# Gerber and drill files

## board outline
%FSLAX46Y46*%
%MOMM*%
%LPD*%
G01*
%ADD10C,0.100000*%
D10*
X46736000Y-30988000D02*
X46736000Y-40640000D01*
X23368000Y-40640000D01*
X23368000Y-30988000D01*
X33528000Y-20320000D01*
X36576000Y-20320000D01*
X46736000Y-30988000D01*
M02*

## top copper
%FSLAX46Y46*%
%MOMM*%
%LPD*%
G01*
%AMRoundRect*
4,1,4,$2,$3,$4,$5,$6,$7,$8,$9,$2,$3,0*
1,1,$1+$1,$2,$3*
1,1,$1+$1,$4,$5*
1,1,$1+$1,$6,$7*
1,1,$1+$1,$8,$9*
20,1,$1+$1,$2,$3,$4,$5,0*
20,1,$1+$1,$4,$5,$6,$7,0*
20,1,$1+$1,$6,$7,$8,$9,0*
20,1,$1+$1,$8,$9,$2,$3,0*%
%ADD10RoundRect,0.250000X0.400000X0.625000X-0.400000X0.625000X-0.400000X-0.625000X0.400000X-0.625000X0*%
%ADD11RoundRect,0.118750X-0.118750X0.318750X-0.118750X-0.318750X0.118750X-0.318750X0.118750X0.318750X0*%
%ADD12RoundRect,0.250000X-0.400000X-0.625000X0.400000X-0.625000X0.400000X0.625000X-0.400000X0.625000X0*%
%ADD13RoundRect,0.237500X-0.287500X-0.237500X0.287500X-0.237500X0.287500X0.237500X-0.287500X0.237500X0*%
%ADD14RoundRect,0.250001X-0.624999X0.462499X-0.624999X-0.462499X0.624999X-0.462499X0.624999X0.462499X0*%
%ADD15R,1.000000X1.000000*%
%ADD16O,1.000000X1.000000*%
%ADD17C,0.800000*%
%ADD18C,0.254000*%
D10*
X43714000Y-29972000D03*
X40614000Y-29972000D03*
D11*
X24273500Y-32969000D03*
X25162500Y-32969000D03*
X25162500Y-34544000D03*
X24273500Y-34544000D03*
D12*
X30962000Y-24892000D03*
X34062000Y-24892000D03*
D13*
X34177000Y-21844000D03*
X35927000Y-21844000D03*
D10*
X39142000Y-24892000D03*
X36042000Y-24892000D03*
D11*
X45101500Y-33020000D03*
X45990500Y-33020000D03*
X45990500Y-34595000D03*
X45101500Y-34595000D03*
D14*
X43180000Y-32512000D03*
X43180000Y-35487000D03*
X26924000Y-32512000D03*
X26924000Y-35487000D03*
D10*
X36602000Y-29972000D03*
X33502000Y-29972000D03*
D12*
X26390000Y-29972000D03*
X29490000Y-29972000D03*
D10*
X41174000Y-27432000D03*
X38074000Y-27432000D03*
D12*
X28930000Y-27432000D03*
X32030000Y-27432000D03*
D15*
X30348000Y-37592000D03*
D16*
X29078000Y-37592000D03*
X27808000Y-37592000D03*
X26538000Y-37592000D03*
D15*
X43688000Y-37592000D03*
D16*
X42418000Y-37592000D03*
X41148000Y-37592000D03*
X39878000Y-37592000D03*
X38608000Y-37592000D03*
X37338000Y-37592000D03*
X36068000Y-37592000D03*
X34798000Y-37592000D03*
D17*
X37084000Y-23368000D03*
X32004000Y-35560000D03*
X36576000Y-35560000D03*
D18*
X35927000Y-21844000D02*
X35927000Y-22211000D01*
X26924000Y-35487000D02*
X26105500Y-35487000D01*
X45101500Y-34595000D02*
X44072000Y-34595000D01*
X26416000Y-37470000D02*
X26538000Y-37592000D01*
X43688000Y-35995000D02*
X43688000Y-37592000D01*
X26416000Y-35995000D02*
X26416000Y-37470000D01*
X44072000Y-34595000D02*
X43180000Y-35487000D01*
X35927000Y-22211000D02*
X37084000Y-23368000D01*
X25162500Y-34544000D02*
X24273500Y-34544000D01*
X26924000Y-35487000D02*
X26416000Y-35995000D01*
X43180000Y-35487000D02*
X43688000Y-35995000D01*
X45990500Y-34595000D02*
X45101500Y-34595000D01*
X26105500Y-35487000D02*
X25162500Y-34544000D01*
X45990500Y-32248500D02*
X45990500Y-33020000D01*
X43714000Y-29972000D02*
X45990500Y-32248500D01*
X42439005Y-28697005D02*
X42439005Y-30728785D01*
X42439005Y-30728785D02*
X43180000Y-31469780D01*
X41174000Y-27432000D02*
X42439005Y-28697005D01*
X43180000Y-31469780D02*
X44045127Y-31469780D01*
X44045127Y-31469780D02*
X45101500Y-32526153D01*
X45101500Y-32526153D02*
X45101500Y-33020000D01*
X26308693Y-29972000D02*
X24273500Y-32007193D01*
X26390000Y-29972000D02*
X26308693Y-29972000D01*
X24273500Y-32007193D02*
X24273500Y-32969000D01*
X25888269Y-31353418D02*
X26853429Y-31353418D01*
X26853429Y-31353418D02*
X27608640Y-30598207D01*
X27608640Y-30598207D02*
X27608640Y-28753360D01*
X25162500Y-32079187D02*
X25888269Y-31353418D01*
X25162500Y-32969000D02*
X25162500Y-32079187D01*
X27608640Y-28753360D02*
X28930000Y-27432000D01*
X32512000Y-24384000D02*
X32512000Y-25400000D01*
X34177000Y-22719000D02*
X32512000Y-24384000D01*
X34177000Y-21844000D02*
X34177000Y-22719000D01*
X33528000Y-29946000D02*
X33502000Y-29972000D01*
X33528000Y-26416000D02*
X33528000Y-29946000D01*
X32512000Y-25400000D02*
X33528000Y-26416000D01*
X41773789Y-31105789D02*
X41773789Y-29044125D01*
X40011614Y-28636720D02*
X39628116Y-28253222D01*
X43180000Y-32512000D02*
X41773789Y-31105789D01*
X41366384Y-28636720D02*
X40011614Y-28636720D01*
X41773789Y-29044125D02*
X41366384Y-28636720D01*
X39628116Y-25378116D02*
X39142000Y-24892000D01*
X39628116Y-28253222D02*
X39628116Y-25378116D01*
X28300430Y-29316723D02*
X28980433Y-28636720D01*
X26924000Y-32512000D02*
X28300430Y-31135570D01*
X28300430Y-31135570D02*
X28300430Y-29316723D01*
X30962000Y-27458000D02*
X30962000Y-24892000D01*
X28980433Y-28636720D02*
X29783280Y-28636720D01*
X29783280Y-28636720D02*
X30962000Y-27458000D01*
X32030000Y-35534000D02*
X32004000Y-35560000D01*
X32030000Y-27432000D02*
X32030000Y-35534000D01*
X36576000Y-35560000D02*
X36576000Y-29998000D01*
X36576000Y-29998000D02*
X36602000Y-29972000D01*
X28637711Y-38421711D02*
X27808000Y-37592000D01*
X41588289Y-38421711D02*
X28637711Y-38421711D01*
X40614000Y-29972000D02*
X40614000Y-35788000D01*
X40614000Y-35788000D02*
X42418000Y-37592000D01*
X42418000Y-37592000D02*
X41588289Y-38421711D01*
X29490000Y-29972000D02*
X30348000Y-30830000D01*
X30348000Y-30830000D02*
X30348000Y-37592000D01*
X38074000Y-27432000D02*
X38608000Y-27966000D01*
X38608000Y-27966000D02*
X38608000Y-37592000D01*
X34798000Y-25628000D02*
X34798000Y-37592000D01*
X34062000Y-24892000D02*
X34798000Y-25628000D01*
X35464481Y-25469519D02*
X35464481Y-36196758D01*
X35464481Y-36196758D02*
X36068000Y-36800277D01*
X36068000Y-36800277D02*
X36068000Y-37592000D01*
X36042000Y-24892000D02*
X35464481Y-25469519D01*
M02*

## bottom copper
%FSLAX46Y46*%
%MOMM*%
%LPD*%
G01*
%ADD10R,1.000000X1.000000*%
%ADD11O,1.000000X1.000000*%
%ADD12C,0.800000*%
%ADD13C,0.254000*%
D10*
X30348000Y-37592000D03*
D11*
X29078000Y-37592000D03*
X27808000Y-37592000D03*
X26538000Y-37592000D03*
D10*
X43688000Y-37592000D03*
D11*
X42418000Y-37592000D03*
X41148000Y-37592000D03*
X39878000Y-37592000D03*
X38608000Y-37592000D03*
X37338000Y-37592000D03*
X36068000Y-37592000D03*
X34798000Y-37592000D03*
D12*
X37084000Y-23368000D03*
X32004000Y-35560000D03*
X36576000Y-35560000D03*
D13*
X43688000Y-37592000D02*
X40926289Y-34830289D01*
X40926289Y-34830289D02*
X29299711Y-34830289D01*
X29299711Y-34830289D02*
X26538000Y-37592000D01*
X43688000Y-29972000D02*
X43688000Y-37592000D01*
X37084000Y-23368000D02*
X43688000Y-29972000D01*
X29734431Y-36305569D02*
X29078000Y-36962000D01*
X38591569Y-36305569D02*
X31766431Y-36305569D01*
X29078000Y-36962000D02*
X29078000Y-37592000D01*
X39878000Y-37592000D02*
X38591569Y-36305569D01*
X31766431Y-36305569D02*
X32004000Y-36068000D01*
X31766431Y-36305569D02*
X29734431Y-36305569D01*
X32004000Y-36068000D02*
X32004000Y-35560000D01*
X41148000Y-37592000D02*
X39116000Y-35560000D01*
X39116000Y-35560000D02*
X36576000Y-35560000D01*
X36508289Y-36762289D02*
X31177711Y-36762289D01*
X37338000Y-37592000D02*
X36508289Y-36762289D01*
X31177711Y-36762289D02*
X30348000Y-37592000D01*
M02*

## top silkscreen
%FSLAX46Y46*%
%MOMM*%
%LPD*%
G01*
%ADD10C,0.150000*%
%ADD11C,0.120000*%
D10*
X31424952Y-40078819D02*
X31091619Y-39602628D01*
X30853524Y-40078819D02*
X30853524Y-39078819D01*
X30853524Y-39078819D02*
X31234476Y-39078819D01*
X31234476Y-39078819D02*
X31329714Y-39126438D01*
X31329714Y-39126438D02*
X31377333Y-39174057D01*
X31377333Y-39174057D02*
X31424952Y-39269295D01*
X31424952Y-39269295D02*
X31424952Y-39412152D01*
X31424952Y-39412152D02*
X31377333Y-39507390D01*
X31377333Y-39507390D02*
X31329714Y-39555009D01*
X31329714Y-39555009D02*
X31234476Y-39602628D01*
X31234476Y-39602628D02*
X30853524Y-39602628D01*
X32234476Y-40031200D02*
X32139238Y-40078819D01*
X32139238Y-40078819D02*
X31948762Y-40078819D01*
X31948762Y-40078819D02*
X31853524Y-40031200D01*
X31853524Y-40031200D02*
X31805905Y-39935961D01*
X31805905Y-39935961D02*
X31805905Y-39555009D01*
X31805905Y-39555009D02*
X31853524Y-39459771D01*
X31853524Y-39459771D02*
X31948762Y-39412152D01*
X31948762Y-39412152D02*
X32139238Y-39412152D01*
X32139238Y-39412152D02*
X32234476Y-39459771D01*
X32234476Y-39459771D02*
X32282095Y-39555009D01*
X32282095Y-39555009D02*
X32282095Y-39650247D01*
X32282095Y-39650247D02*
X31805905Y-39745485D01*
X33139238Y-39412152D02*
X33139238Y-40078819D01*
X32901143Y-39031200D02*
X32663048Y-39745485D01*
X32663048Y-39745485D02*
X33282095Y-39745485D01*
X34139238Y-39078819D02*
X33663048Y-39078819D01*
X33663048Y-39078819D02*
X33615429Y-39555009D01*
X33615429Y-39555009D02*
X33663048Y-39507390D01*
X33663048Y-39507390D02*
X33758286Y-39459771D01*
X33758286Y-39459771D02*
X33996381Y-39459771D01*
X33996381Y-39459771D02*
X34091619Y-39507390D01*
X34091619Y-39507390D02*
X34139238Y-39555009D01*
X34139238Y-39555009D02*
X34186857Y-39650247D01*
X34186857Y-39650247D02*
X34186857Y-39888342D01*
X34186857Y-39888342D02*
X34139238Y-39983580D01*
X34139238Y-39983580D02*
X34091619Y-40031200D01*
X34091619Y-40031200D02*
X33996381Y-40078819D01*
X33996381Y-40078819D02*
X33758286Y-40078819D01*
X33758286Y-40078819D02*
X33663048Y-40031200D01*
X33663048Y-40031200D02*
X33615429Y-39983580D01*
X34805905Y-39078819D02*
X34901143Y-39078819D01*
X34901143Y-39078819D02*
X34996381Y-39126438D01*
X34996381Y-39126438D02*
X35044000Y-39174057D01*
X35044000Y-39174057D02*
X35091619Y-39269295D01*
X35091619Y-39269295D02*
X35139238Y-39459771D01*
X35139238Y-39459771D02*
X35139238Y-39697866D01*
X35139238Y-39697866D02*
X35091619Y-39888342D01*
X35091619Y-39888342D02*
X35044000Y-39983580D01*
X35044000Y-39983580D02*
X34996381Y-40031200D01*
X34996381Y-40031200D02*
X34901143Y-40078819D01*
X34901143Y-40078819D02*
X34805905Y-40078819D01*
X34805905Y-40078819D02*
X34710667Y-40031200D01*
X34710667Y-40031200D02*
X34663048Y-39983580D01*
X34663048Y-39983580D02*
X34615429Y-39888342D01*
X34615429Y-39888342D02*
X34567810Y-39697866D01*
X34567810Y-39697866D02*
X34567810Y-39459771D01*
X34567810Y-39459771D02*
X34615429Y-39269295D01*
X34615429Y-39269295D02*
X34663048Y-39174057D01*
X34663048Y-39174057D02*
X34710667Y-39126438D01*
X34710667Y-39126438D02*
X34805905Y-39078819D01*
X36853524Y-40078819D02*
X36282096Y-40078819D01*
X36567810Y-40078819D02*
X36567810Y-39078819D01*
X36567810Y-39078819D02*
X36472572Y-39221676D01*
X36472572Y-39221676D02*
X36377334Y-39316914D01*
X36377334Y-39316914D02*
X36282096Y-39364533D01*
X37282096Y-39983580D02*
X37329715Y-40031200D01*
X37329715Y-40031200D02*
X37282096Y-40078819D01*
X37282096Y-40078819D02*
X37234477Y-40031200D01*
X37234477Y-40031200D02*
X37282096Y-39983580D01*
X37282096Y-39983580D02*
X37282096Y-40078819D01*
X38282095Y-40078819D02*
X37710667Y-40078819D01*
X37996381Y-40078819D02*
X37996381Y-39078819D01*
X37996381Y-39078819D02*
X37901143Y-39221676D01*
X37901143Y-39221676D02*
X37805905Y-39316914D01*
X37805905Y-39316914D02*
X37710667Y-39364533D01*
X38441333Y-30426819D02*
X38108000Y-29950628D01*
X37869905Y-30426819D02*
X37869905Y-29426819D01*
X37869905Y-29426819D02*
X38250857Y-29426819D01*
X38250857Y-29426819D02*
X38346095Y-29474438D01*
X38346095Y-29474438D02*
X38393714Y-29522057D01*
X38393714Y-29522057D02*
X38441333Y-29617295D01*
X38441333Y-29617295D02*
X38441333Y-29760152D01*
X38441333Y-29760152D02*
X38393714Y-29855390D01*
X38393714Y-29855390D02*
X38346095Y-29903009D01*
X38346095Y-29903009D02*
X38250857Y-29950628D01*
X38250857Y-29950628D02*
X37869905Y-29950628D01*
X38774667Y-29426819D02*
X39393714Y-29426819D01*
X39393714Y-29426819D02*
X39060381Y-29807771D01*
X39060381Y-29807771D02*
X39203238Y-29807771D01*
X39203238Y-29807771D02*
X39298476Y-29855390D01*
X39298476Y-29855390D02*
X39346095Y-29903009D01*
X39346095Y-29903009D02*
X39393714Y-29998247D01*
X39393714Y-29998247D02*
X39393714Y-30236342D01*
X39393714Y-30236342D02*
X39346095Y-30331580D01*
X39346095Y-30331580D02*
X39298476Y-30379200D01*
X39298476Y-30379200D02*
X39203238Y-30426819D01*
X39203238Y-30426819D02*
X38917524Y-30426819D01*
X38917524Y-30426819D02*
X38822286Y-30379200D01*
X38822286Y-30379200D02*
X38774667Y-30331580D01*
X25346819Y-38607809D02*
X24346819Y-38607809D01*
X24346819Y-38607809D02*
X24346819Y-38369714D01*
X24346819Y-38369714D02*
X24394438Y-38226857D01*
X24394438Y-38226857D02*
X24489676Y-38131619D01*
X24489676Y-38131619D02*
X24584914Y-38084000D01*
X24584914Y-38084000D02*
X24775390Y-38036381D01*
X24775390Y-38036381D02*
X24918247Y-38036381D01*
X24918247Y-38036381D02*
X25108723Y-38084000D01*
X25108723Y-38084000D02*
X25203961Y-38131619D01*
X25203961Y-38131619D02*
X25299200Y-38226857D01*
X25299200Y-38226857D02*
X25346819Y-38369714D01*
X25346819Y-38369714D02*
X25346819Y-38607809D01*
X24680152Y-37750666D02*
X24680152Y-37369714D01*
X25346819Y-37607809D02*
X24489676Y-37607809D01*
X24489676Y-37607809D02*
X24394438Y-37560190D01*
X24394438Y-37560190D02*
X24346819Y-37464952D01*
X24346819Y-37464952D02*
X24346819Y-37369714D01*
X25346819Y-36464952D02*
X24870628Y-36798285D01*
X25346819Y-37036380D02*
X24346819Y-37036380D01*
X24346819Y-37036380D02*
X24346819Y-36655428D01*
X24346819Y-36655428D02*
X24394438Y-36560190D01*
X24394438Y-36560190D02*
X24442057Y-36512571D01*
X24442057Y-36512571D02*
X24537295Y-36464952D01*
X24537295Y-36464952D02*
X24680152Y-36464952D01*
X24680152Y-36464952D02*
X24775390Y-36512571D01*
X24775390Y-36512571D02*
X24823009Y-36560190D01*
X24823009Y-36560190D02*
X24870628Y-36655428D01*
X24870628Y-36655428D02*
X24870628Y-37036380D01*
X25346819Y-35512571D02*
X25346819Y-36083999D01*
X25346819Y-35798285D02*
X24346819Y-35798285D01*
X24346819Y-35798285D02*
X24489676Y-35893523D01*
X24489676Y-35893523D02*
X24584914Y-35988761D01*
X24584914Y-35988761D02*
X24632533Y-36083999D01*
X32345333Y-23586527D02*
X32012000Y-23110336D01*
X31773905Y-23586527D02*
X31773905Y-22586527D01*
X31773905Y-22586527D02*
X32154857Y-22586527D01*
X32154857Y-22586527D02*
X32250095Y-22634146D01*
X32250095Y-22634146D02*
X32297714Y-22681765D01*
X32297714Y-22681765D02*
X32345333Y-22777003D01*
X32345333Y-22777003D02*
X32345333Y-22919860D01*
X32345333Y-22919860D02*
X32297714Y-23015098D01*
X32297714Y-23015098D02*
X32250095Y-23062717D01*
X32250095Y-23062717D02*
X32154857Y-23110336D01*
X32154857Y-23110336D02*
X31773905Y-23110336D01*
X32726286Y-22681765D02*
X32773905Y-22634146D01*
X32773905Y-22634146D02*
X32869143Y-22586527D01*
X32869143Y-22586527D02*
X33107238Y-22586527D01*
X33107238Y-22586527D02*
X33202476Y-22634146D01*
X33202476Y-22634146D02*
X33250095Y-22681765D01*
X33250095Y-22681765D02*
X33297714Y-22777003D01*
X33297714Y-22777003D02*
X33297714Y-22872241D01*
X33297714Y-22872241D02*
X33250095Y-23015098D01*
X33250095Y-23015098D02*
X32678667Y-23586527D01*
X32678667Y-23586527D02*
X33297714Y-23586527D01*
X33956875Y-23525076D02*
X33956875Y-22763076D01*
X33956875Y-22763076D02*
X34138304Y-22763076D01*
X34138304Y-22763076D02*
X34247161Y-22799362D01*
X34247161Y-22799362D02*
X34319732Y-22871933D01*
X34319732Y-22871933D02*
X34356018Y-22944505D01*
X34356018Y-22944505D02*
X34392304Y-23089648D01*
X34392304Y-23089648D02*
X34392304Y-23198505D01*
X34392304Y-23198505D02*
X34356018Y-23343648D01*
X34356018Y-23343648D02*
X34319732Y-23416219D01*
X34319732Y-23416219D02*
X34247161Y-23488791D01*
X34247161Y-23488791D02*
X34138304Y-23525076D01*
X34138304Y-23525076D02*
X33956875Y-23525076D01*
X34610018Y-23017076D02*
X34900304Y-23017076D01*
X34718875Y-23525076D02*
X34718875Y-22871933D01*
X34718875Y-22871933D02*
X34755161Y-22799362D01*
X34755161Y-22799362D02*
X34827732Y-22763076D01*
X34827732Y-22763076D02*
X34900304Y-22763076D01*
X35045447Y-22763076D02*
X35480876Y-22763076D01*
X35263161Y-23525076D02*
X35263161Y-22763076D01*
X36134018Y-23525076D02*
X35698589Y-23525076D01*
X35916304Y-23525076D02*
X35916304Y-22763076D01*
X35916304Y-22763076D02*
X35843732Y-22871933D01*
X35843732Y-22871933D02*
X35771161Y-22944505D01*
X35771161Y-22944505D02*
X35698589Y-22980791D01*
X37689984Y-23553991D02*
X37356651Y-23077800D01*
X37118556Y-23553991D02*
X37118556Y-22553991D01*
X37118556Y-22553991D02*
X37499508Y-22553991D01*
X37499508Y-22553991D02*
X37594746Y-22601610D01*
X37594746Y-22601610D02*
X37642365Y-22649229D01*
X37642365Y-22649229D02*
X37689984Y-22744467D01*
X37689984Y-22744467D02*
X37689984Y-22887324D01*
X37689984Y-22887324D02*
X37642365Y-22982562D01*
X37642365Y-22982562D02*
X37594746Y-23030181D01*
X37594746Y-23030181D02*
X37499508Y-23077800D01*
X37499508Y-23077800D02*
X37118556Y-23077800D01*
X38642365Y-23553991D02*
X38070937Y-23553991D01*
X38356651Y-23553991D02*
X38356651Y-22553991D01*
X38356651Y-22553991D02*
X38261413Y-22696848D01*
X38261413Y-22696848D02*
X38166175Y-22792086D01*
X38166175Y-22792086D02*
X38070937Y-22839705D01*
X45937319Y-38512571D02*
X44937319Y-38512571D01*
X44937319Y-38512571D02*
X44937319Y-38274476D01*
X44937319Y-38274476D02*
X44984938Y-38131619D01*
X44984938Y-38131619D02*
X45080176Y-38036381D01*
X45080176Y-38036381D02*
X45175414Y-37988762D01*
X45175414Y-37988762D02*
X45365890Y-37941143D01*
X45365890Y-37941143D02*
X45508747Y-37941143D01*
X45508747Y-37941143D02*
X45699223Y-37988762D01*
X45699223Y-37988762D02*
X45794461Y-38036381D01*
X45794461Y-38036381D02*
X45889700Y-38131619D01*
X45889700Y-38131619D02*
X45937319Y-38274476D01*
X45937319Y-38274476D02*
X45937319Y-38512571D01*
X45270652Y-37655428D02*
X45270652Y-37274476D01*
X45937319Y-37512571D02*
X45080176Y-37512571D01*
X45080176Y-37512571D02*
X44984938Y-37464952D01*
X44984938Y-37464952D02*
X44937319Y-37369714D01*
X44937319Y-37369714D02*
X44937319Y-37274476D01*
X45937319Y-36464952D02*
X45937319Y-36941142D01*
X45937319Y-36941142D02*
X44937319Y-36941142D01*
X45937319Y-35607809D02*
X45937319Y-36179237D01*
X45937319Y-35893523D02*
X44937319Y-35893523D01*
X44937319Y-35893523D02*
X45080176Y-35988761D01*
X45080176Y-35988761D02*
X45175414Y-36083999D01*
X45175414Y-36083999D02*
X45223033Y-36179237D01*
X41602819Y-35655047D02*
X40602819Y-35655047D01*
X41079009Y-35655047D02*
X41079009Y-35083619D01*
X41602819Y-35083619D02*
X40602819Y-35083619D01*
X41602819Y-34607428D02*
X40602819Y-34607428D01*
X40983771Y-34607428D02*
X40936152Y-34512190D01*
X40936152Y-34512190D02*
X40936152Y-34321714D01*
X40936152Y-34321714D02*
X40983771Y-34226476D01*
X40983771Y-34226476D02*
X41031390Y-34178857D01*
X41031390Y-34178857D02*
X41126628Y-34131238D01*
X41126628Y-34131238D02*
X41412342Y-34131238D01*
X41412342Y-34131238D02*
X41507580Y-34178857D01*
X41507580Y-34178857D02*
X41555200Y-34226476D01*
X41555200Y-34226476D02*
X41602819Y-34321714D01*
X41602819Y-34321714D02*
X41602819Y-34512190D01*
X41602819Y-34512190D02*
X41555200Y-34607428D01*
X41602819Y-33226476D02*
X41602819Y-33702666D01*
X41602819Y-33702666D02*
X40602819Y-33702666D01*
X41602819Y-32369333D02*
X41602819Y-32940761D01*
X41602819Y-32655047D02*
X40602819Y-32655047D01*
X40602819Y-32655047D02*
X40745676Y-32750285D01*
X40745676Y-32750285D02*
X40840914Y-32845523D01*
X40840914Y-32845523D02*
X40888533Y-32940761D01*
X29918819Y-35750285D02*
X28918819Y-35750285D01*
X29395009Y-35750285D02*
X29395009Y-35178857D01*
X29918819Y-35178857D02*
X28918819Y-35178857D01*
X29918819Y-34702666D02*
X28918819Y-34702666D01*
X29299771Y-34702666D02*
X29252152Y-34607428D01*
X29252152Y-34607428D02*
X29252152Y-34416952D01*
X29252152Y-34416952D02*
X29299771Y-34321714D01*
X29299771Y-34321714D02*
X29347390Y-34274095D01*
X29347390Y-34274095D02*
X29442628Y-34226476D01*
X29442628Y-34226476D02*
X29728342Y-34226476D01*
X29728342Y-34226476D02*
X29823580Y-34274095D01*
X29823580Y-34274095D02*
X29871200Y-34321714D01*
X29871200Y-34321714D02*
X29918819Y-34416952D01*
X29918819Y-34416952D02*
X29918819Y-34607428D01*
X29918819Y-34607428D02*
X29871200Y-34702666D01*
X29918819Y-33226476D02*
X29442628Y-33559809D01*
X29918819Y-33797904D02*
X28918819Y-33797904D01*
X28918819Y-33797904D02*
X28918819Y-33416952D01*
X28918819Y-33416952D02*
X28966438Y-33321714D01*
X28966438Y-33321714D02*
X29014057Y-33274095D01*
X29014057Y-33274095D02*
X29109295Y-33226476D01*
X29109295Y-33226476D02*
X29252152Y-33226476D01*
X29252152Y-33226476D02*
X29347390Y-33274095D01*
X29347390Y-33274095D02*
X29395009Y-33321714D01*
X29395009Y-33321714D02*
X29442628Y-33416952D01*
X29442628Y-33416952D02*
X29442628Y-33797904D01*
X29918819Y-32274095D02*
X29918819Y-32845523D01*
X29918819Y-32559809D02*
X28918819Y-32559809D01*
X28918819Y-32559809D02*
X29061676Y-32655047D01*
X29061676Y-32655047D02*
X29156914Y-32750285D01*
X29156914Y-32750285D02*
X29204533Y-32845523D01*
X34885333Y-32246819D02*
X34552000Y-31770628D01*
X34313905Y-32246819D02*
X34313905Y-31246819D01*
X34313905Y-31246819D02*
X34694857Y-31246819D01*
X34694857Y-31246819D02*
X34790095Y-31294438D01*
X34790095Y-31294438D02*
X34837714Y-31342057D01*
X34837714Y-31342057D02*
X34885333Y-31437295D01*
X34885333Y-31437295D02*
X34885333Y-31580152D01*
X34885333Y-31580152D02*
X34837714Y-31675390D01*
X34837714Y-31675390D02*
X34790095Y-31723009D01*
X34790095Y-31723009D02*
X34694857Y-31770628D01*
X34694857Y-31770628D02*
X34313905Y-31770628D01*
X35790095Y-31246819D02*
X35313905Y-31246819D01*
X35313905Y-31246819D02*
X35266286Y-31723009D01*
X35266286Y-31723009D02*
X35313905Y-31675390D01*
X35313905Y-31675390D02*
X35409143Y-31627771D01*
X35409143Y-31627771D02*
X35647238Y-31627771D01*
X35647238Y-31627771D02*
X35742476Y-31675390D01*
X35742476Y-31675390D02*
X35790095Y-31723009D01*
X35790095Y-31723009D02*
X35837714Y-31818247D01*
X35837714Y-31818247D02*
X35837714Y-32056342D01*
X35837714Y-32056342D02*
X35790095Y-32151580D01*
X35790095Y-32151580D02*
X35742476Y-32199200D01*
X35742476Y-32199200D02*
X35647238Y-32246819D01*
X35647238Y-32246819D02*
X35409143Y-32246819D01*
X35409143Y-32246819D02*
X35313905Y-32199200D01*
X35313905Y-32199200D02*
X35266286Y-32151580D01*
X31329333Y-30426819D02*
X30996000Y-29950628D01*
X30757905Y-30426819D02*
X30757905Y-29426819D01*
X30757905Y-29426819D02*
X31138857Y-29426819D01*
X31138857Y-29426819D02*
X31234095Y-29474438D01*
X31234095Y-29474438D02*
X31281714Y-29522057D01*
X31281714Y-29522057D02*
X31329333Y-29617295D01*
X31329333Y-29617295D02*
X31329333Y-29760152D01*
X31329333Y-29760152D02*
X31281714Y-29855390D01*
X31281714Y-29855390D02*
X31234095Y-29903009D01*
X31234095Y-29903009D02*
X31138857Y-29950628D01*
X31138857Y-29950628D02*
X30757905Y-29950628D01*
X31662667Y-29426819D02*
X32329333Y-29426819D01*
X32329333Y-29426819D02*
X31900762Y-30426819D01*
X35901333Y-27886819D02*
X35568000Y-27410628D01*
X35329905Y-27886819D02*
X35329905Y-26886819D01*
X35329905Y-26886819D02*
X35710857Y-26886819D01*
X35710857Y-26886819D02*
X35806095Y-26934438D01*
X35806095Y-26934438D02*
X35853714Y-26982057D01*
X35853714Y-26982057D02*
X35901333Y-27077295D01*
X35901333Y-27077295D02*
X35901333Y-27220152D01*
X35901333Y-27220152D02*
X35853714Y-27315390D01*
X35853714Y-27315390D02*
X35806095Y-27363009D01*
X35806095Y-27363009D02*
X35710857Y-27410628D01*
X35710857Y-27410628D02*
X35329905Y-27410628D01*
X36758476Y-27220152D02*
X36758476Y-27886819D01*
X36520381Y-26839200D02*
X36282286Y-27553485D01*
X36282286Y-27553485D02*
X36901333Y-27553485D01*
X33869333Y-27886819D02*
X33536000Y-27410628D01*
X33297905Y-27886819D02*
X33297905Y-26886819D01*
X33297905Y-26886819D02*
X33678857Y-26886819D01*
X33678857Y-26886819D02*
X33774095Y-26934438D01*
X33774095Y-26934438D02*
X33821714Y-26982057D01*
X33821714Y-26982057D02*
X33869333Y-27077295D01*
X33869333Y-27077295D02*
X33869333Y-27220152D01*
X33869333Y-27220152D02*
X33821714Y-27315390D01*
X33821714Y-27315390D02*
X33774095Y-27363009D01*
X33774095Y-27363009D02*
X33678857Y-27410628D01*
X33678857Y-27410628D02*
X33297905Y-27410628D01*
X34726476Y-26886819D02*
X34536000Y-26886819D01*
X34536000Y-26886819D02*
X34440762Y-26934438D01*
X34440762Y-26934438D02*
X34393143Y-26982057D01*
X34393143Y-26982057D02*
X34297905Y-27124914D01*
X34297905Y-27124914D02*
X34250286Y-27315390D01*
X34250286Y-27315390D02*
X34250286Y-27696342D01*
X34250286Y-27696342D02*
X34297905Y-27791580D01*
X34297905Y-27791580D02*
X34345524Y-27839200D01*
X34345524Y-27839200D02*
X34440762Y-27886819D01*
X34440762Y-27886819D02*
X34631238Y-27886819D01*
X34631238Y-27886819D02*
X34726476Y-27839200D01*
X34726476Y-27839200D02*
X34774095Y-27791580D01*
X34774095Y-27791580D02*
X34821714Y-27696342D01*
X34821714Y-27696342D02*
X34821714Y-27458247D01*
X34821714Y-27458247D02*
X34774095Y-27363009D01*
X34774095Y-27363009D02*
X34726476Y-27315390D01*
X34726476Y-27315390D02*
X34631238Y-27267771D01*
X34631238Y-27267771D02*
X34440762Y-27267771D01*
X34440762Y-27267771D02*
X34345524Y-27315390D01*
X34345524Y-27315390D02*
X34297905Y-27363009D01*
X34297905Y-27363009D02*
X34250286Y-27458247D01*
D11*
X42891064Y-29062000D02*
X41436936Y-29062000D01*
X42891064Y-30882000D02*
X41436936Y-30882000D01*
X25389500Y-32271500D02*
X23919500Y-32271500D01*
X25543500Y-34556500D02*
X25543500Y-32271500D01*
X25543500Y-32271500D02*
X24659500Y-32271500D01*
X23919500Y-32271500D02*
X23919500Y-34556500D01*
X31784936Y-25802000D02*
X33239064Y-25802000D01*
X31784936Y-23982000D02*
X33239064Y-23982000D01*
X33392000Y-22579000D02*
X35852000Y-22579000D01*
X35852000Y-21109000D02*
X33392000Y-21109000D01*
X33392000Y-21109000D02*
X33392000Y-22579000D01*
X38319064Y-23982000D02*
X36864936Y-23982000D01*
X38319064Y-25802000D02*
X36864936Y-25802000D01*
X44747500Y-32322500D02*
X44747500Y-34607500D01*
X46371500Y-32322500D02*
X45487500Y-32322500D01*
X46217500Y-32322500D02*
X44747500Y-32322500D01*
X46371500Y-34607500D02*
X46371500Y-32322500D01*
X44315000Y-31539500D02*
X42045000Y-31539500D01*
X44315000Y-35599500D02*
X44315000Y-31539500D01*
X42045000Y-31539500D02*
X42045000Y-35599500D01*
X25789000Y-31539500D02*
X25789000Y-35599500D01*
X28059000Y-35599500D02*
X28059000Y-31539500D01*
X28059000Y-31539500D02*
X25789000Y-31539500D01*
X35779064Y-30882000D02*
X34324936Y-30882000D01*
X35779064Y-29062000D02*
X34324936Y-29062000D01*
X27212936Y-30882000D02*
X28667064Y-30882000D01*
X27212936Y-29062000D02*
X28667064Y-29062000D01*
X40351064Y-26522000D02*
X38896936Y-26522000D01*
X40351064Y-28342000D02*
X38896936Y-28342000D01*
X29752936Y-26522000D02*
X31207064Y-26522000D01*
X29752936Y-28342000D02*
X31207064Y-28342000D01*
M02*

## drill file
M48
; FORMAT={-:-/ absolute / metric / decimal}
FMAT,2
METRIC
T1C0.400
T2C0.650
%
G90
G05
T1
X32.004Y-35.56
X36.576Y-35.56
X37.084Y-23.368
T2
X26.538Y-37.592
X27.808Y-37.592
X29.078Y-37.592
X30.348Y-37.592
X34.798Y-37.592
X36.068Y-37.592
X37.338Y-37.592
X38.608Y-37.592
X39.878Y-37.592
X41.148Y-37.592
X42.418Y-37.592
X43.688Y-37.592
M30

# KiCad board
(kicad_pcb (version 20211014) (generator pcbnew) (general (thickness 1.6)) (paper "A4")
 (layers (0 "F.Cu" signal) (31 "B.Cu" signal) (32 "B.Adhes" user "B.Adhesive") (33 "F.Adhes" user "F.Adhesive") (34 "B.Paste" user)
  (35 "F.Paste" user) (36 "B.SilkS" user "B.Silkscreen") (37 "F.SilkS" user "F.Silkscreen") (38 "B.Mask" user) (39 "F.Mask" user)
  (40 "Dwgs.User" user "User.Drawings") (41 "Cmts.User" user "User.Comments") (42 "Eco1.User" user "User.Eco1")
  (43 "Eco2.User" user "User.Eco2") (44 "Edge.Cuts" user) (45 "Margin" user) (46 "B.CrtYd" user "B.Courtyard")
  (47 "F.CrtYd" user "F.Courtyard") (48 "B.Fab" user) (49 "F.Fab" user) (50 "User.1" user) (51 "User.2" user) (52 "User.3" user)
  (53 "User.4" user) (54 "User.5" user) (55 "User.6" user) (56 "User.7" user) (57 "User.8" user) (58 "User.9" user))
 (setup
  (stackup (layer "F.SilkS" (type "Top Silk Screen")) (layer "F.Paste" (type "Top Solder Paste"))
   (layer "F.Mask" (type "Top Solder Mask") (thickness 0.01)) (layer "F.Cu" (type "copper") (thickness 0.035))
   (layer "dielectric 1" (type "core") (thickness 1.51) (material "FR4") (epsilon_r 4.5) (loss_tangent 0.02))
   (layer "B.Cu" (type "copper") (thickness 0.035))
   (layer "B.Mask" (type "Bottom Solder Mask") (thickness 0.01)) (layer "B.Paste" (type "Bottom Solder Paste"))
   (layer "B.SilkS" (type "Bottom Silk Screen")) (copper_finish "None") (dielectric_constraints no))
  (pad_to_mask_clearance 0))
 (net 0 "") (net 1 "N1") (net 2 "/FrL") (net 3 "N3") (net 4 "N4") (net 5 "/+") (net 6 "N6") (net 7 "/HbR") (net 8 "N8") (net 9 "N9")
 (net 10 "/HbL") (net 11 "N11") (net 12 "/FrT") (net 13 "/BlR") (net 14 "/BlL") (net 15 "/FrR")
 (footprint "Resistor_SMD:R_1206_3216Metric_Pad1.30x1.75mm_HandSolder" (layer "F.Cu") (at 42.164 29.972 180)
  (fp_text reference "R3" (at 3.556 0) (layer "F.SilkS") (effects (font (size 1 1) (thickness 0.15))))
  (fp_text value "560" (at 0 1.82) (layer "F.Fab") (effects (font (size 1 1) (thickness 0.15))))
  (fp_line (start -0.727064 0.91) (end 0.727064 0.91) (layer "F.SilkS") (width 0.12))
  (fp_line (start -0.727064 -0.91) (end 0.727064 -0.91) (layer "F.SilkS") (width 0.12))
  (pad "1" smd roundrect (at -1.55 0 180) (size 1.3 1.75) (layers "F.Cu" "F.Paste" "F.Mask") (roundrect_rratio 0.192308) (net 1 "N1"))
  (pad "2" smd roundrect (at 1.55 0 180) (size 1.3 1.75) (layers "F.Cu" "F.Paste" "F.Mask") (roundrect_rratio 0.192308) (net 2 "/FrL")))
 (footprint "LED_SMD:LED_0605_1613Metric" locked (layer "F.Cu") (at 24.6545 33.7565 -90)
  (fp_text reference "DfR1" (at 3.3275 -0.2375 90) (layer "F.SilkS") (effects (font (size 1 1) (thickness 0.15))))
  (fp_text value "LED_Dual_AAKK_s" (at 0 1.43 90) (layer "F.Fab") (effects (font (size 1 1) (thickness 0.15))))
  (fp_line (start -1.485 -0.735) (end -1.485 0.735) (layer "F.SilkS") (width 0.12))
  (fp_line (start 0.8 -0.889) (end -1.485 -0.889) (layer "F.SilkS") (width 0.12))
  (fp_line (start -1.485 -0.889) (end -1.485 -0.005) (layer "F.SilkS") (width 0.12))
  (fp_line (start -1.485 0.735) (end 0.8 0.735) (layer "F.SilkS") (width 0.12))
  (pad "1" smd roundrect locked (at -0.7875 0.381 270) (size 0.875 0.475) (layers "F.Cu" "F.Paste" "F.Mask") (roundrect_rratio 0.25)
   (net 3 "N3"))
  (pad "2" smd roundrect locked (at -0.7875 -0.508 270) (size 0.875 0.475) (layers "F.Cu" "F.Paste" "F.Mask") (roundrect_rratio 0.25)
   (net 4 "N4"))
  (pad "3" smd roundrect locked (at 0.7875 -0.508 270) (size 0.875 0.475) (layers "F.Cu" "F.Paste" "F.Mask") (roundrect_rratio 0.25)
   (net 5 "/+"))
  (pad "4" smd roundrect locked (at 0.7875 0.381 270) (size 0.875 0.475) (layers "F.Cu" "F.Paste" "F.Mask") (roundrect_rratio 0.25)
   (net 5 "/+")))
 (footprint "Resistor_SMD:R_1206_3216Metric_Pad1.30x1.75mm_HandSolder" (layer "F.Cu") (at 32.512 24.892)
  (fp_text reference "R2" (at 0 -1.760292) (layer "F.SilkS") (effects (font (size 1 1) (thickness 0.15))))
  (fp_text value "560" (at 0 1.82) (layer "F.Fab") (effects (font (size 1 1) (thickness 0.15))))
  (fp_line (start -0.727064 0.91) (end 0.727064 0.91) (layer "F.SilkS") (width 0.12))
  (fp_line (start -0.727064 -0.91) (end 0.727064 -0.91) (layer "F.SilkS") (width 0.12))
  (pad "1" smd roundrect (at -1.55 0) (size 1.3 1.75) (layers "F.Cu" "F.Paste" "F.Mask") (roundrect_rratio 0.192308) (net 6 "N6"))
  (pad "2" smd roundrect (at 1.55 0) (size 1.3 1.75) (layers "F.Cu" "F.Paste" "F.Mask") (roundrect_rratio 0.192308) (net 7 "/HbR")))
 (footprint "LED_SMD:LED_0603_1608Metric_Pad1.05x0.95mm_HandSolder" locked (layer "F.Cu") (at 35.052 21.844)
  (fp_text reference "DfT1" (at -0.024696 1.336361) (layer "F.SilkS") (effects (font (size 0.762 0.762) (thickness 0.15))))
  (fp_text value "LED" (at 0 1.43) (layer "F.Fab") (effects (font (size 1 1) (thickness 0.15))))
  (fp_line (start -1.66 0.735) (end 0.8 0.735) (layer "F.SilkS") (width 0.12))
  (fp_line (start 0.8 -0.735) (end -1.66 -0.735) (layer "F.SilkS") (width 0.12))
  (fp_line (start -1.66 -0.735) (end -1.66 0.735) (layer "F.SilkS") (width 0.12))
  (pad "1" smd roundrect locked (at -0.875 0) (size 1.05 0.95) (layers "F.Cu" "F.Paste" "F.Mask") (roundrect_rratio 0.25) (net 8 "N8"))
  (pad "2" smd roundrect locked (at 0.875 0) (size 1.05 0.95) (layers "F.Cu" "F.Paste" "F.Mask") (roundrect_rratio 0.25) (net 5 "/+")))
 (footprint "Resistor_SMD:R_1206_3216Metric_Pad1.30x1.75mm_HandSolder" (layer "F.Cu") (at 37.592 24.892 180)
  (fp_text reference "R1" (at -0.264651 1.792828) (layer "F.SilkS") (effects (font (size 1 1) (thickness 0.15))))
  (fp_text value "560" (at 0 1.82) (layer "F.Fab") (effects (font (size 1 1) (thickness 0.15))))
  (fp_line (start -0.727064 0.91) (end 0.727064 0.91) (layer "F.SilkS") (width 0.12))
  (fp_line (start -0.727064 -0.91) (end 0.727064 -0.91) (layer "F.SilkS") (width 0.12))
  (pad "1" smd roundrect (at -1.55 0 180) (size 1.3 1.75) (layers "F.Cu" "F.Paste" "F.Mask") (roundrect_rratio 0.192308) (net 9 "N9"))
  (pad "2" smd roundrect (at 1.55 0 180) (size 1.3 1.75) (layers "F.Cu" "F.Paste" "F.Mask") (roundrect_rratio 0.192308) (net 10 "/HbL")))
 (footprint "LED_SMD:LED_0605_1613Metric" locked (layer "F.Cu") (at 45.4825 33.8075 -90)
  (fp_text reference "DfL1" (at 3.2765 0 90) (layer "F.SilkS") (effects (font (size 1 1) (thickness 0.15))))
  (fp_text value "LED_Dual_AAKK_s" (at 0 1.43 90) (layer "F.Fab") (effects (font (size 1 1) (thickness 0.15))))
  (fp_line (start -1.485 0.735) (end 0.8 0.735) (layer "F.SilkS") (width 0.12))
  (fp_line (start -1.485 -0.889) (end -1.485 -0.005) (layer "F.SilkS") (width 0.12))
  (fp_line (start -1.485 -0.735) (end -1.485 0.735) (layer "F.SilkS") (width 0.12))
  (fp_line (start 0.8 -0.889) (end -1.485 -0.889) (layer "F.SilkS") (width 0.12))
  (pad "1" smd roundrect locked (at -0.7875 0.381 270) (size 0.875 0.475) (layers "F.Cu" "F.Paste" "F.Mask") (roundrect_rratio 0.25)
   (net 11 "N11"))
  (pad "2" smd roundrect locked (at -0.7875 -0.508 270) (size 0.875 0.475) (layers "F.Cu" "F.Paste" "F.Mask") (roundrect_rratio 0.25)
   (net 1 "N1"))
  (pad "3" smd roundrect locked (at 0.7875 -0.508 270) (size 0.875 0.475) (layers "F.Cu" "F.Paste" "F.Mask") (roundrect_rratio 0.25)
   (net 5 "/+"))
  (pad "4" smd roundrect locked (at 0.7875 0.381 270) (size 0.875 0.475) (layers "F.Cu" "F.Paste" "F.Mask") (roundrect_rratio 0.25)
   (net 5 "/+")))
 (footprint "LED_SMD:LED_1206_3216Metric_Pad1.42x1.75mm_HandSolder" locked (layer "F.Cu") (at 43.18 33.9995 -90)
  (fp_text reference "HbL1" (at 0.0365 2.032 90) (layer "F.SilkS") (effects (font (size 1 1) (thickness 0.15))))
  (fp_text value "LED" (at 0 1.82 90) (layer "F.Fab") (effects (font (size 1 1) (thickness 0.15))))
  (fp_line (start -2.46 -1.135) (end -2.46 1.135) (layer "F.SilkS") (width 0.12))
  (fp_line (start 1.6 -1.135) (end -2.46 -1.135) (layer "F.SilkS") (width 0.12))
  (fp_line (start -2.46 1.135) (end 1.6 1.135) (layer "F.SilkS") (width 0.12))
  (pad "1" smd roundrect locked (at -1.4875 0 270) (size 1.425 1.75) (layers "F.Cu" "F.Paste" "F.Mask") (roundrect_rratio 0.1754392982)
   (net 9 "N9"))
  (pad "2" smd roundrect locked (at 1.4875 0 270) (size 1.425 1.75) (layers "F.Cu" "F.Paste" "F.Mask") (roundrect_rratio 0.1754392982)
   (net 5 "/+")))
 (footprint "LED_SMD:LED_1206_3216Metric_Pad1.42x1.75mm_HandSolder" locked (layer "F.Cu") (at 26.924 33.9995 -90)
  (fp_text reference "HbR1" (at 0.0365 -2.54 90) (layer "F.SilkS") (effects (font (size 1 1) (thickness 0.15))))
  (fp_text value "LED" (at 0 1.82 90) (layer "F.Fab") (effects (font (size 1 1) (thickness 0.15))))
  (fp_line (start -2.46 1.135) (end 1.6 1.135) (layer "F.SilkS") (width 0.12))
  (fp_line (start 1.6 -1.135) (end -2.46 -1.135) (layer "F.SilkS") (width 0.12))
  (fp_line (start -2.46 -1.135) (end -2.46 1.135) (layer "F.SilkS") (width 0.12))
  (pad "1" smd roundrect locked (at -1.4875 0 270) (size 1.425 1.75) (layers "F.Cu" "F.Paste" "F.Mask") (roundrect_rratio 0.1754392982)
   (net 6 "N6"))
  (pad "2" smd roundrect locked (at 1.4875 0 270) (size 1.425 1.75) (layers "F.Cu" "F.Paste" "F.Mask") (roundrect_rratio 0.1754392982)
   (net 5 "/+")))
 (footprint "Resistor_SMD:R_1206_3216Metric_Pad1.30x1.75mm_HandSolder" (layer "F.Cu") (at 35.052 29.972 180)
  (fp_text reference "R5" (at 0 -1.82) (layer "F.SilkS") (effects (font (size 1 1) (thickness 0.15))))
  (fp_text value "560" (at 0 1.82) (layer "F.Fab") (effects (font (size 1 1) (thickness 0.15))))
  (fp_line (start -0.727064 -0.91) (end 0.727064 -0.91) (layer "F.SilkS") (width 0.12))
  (fp_line (start -0.727064 0.91) (end 0.727064 0.91) (layer "F.SilkS") (width 0.12))
  (pad "1" smd roundrect (at -1.55 0 180) (size 1.3 1.75) (layers "F.Cu" "F.Paste" "F.Mask") (roundrect_rratio 0.192308) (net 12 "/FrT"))
  (pad "2" smd roundrect (at 1.55 0 180) (size 1.3 1.75) (layers "F.Cu" "F.Paste" "F.Mask") (roundrect_rratio 0.192308) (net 8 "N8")))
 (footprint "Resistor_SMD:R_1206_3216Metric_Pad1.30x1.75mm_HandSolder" (layer "F.Cu") (at 27.94 29.972)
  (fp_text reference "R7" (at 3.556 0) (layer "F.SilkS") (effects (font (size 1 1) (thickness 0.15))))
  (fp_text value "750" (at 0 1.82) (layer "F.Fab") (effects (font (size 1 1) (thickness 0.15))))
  (fp_line (start -0.727064 0.91) (end 0.727064 0.91) (layer "F.SilkS") (width 0.12))
  (fp_line (start -0.727064 -0.91) (end 0.727064 -0.91) (layer "F.SilkS") (width 0.12))
  (pad "1" smd roundrect (at -1.55 0) (size 1.3 1.75) (layers "F.Cu" "F.Paste" "F.Mask") (roundrect_rratio 0.192308) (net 3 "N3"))
  (pad "2" smd roundrect (at 1.55 0) (size 1.3 1.75) (layers "F.Cu" "F.Paste" "F.Mask") (roundrect_rratio 0.192308) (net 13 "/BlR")))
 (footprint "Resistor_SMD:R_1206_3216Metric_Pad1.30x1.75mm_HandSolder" (layer "F.Cu") (at 39.624 27.432 180)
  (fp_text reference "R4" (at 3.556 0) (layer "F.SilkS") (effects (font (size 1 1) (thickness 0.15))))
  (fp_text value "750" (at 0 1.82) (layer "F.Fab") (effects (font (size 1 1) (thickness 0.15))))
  (fp_line (start -0.727064 0.91) (end 0.727064 0.91) (layer "F.SilkS") (width 0.12))
  (fp_line (start -0.727064 -0.91) (end 0.727064 -0.91) (layer "F.SilkS") (width 0.12))
  (pad "1" smd roundrect (at -1.55 0 180) (size 1.3 1.75) (layers "F.Cu" "F.Paste" "F.Mask") (roundrect_rratio 0.192308) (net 11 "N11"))
  (pad "2" smd roundrect (at 1.55 0 180) (size 1.3 1.75) (layers "F.Cu" "F.Paste" "F.Mask") (roundrect_rratio 0.192308) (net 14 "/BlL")))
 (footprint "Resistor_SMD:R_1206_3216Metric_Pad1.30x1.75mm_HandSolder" (layer "F.Cu") (at 30.48 27.432)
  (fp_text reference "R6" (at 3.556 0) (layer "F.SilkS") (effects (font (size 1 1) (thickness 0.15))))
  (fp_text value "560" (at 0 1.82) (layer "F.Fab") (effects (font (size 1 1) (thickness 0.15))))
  (fp_line (start -0.727064 -0.91) (end 0.727064 -0.91) (layer "F.SilkS") (width 0.12))
  (fp_line (start -0.727064 0.91) (end 0.727064 0.91) (layer "F.SilkS") (width 0.12))
  (pad "1" smd roundrect (at -1.55 0) (size 1.3 1.75) (layers "F.Cu" "F.Paste" "F.Mask") (roundrect_rratio 0.192308) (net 4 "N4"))
  (pad "2" smd roundrect (at 1.55 0) (size 1.3 1.75) (layers "F.Cu" "F.Paste" "F.Mask") (roundrect_rratio 0.192308) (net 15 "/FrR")))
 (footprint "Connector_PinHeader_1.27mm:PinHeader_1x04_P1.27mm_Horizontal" (layer "B.Cu") (at 30.348 37.592 90)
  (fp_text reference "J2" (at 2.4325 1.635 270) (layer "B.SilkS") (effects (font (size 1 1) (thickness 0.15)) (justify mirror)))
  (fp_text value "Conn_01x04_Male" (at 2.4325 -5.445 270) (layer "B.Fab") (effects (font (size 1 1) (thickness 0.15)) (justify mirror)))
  (pad "1" thru_hole rect (at 0 0 90) (size 1 1) (drill 0.65) (layers *.Cu *.Mask) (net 13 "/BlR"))
  (pad "2" thru_hole oval (at 0 -1.27 90) (size 1 1) (drill 0.65) (layers *.Cu *.Mask) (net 15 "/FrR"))
  (pad "3" thru_hole oval (at 0 -2.54 90) (size 1 1) (drill 0.65) (layers *.Cu *.Mask) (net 2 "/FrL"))
  (pad "4" thru_hole oval (at 0 -3.81 90) (size 1 1) (drill 0.65) (layers *.Cu *.Mask) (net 5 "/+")))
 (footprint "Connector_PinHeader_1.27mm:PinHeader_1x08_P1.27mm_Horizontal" (layer "B.Cu") (at 43.688 37.592 90)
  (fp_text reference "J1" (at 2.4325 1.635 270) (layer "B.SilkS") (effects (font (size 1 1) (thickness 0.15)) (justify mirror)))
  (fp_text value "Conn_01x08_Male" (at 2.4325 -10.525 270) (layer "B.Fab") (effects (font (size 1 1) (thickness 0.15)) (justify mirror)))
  (pad "1" thru_hole rect (at 0 0 90) (size 1 1) (drill 0.65) (layers *.Cu *.Mask) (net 5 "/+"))
  (pad "2" thru_hole oval (at 0 -1.27 90) (size 1 1) (drill 0.65) (layers *.Cu *.Mask) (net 2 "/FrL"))
  (pad "3" thru_hole oval (at 0 -2.54 90) (size 1 1) (drill 0.65) (layers *.Cu *.Mask) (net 12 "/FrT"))
  (pad "4" thru_hole oval (at 0 -3.81 90) (size 1 1) (drill 0.65) (layers *.Cu *.Mask) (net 15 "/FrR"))
  (pad "5" thru_hole oval (at 0 -5.08 90) (size 1 1) (drill 0.65) (layers *.Cu *.Mask) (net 14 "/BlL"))
  (pad "6" thru_hole oval (at 0 -6.35 90) (size 1 1) (drill 0.65) (layers *.Cu *.Mask) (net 13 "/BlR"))
  (pad "7" thru_hole oval (at 0 -7.62 90) (size 1 1) (drill 0.65) (layers *.Cu *.Mask) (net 10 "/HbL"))
  (pad "8" thru_hole oval (at 0 -8.89 90) (size 1 1) (drill 0.65) (layers *.Cu *.Mask) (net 7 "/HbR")))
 (gr_poly locked
  (pts (xy 46.736 30.988) (xy 46.736 40.64) (xy 23.368 40.64) (xy 23.368 30.988) (xy 33.528 20.32) (xy 36.576 20.32)) (layer "Edge.Cuts")
  (width 0.1) (fill none))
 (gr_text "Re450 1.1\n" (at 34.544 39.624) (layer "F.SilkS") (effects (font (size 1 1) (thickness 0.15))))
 (segment (start 35.927 21.844) (end 35.927 22.211) (width 0.254) (layer "F.Cu") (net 5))
 (segment (start 26.924 35.487) (end 26.1055 35.487) (width 0.254) (layer "F.Cu") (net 5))
 (segment (start 45.1015 34.595) (end 44.072 34.595) (width 0.254) (layer "F.Cu") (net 5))
 (segment (start 26.416 37.47) (end 26.538 37.592) (width 0.254) (layer "F.Cu") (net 5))
 (segment (start 43.688 35.995) (end 43.688 37.592) (width 0.254) (layer "F.Cu") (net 5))
 (segment (start 26.416 35.995) (end 26.416 37.47) (width 0.254) (layer "F.Cu") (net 5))
 (segment (start 44.072 34.595) (end 43.18 35.487) (width 0.254) (layer "F.Cu") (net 5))
 (segment (start 35.927 22.211) (end 37.084 23.368) (width 0.254) (layer "F.Cu") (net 5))
 (segment (start 25.1625 34.544) (end 24.2735 34.544) (width 0.254) (layer "F.Cu") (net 5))
 (segment (start 26.924 35.487) (end 26.416 35.995) (width 0.254) (layer "F.Cu") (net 5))
 (segment (start 43.18 35.487) (end 43.688 35.995) (width 0.254) (layer "F.Cu") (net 5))
 (segment (start 45.9905 34.595) (end 45.1015 34.595) (width 0.254) (layer "F.Cu") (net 5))
 (segment (start 26.1055 35.487) (end 25.1625 34.544) (width 0.254) (layer "F.Cu") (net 5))
 (via (at 37.084 23.368) (size 0.8) (drill 0.4) (layers "F.Cu" "B.Cu") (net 5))
 (segment (start 43.688 37.592) (end 40.926289 34.830289) (width 0.254) (layer "B.Cu") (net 5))
 (segment (start 40.926289 34.830289) (end 29.299711 34.830289) (width 0.254) (layer "B.Cu") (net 5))
 (segment (start 29.299711 34.830289) (end 26.538 37.592) (width 0.254) (layer "B.Cu") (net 5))
 (segment (start 43.688 29.972) (end 43.688 37.592) (width 0.254) (layer "B.Cu") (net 5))
 (segment (start 37.084 23.368) (end 43.688 29.972) (width 0.254) (layer "B.Cu") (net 5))
 (segment (start 45.9905 32.2485) (end 45.9905 33.02) (width 0.254) (layer "F.Cu") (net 1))
 (segment (start 43.714 29.972) (end 45.9905 32.2485) (width 0.254) (layer "F.Cu") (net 1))
 (segment (start 42.439005 28.697005) (end 42.439005 30.728785) (width 0.254) (layer "F.Cu") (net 11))
 (segment (start 42.439005 30.728785) (end 43.18 31.46978) (width 0.254) (layer "F.Cu") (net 11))
 (segment (start 41.174 27.432) (end 42.439005 28.697005) (width 0.254) (layer "F.Cu") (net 11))
 (segment (start 43.18 31.46978) (end 44.045127 31.46978) (width 0.254) (layer "F.Cu") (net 11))
 (segment (start 44.045127 31.46978) (end 45.1015 32.526153) (width 0.254) (layer "F.Cu") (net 11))
 (segment (start 45.1015 32.526153) (end 45.1015 33.02) (width 0.254) (layer "F.Cu") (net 11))
 (segment (start 26.308693 29.972) (end 24.2735 32.007193) (width 0.254) (layer "F.Cu") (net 3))
 (segment (start 26.39 29.972) (end 26.308693 29.972) (width 0.254) (layer "F.Cu") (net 3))
 (segment (start 24.2735 32.007193) (end 24.2735 32.969) (width 0.254) (layer "F.Cu") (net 3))
 (segment (start 25.888269 31.353418) (end 26.853429 31.353418) (width 0.254) (layer "F.Cu") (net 4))
 (segment (start 26.853429 31.353418) (end 27.60864 30.598207) (width 0.254) (layer "F.Cu") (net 4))
 (segment (start 27.60864 30.598207) (end 27.60864 28.75336) (width 0.254) (layer "F.Cu") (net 4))
 (segment (start 25.1625 32.079187) (end 25.888269 31.353418) (width 0.254) (layer "F.Cu") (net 4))
 (segment (start 25.1625 32.969) (end 25.1625 32.079187) (width 0.254) (layer "F.Cu") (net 4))
 (segment (start 27.60864 28.75336) (end 28.93 27.432) (width 0.254) (layer "F.Cu") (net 4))
 (segment (start 32.512 24.384) (end 32.512 25.4) (width 0.254) (layer "F.Cu") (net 8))
 (segment (start 34.177 22.719) (end 32.512 24.384) (width 0.254) (layer "F.Cu") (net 8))
 (segment (start 34.177 21.844) (end 34.177 22.719) (width 0.254) (layer "F.Cu") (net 8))
 (segment (start 33.528 29.946) (end 33.502 29.972) (width 0.254) (layer "F.Cu") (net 8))
 (segment (start 33.528 26.416) (end 33.528 29.946) (width 0.254) (layer "F.Cu") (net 8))
 (segment (start 32.512 25.4) (end 33.528 26.416) (width 0.254) (layer "F.Cu") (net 8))
 (segment (start 41.773789 31.105789) (end 41.773789 29.044125) (width 0.254) (layer "F.Cu") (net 9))
 (segment (start 40.011614 28.63672) (end 39.628116 28.253222) (width 0.254) (layer "F.Cu") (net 9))
 (segment (start 43.18 32.512) (end 41.773789 31.105789) (width 0.254) (layer "F.Cu") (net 9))
 (segment (start 41.366384 28.63672) (end 40.011614 28.63672) (width 0.254) (layer "F.Cu") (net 9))
 (segment (start 41.773789 29.044125) (end 41.366384 28.63672) (width 0.254) (layer "F.Cu") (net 9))
 (segment (start 39.628116 25.378116) (end 39.142 24.892) (width 0.254) (layer "F.Cu") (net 9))
 (segment (start 39.628116 28.253222) (end 39.628116 25.378116) (width 0.254) (layer "F.Cu") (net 9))
 (segment (start 28.30043 29.316723) (end 28.980433 28.63672) (width 0.254) (layer "F.Cu") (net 6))
 (segment (start 26.924 32.512) (end 28.30043 31.13557) (width 0.254) (layer "F.Cu") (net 6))
 (segment (start 28.30043 31.13557) (end 28.30043 29.316723) (width 0.254) (layer "F.Cu") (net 6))
 (segment (start 30.962 27.458) (end 30.962 24.892) (width 0.254) (layer "F.Cu") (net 6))
 (segment (start 28.980433 28.63672) (end 29.78328 28.63672) (width 0.254) (layer "F.Cu") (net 6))
 (segment (start 29.78328 28.63672) (end 30.962 27.458) (width 0.254) (layer "F.Cu") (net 6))
 (segment (start 32.03 35.534) (end 32.004 35.56) (width 0.254) (layer "F.Cu") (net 15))
 (segment (start 32.03 27.432) (end 32.03 35.534) (width 0.254) (layer "F.Cu") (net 15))
 (via (at 32.004 35.56) (size 0.8) (drill 0.4) (layers "F.Cu" "B.Cu") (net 15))
 (segment (start 29.734431 36.305569) (end 29.078 36.962) (width 0.254) (layer "B.Cu") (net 15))
 (segment (start 38.591569 36.305569) (end 31.766431 36.305569) (width 0.254) (layer "B.Cu") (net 15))
 (segment (start 29.078 36.962) (end 29.078 37.592) (width 0.254) (layer "B.Cu") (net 15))
 (segment (start 39.878 37.592) (end 38.591569 36.305569) (width 0.254) (layer "B.Cu") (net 15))
 (segment (start 31.766431 36.305569) (end 32.004 36.068) (width 0.254) (layer "B.Cu") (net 15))
 (segment (start 31.766431 36.305569) (end 29.734431 36.305569) (width 0.254) (layer "B.Cu") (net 15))
 (segment (start 32.004 36.068) (end 32.004 35.56) (width 0.254) (layer "B.Cu") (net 15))
 (segment (start 36.576 35.56) (end 36.576 29.998) (width 0.254) (layer "F.Cu") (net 12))
 (segment (start 36.576 29.998) (end 36.602 29.972) (width 0.254) (layer "F.Cu") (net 12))
 (via (at 36.576 35.56) (size 0.8) (drill 0.4) (layers "F.Cu" "B.Cu") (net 12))
 (segment (start 41.148 37.592) (end 39.116 35.56) (width 0.254) (layer "B.Cu") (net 12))
 (segment (start 39.116 35.56) (end 36.576 35.56) (width 0.254) (layer "B.Cu") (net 12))
 (segment (start 28.637711 38.421711) (end 27.808 37.592) (width 0.254) (layer "F.Cu") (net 2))
 (segment (start 41.588289 38.421711) (end 28.637711 38.421711) (width 0.254) (layer "F.Cu") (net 2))
 (segment (start 40.614 29.972) (end 40.614 35.788) (width 0.254) (layer "F.Cu") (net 2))
 (segment (start 40.614 35.788) (end 42.418 37.592) (width 0.254) (layer "F.Cu") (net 2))
 (segment (start 42.418 37.592) (end 41.588289 38.421711) (width 0.254) (layer "F.Cu") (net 2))
 (segment (start 29.49 29.972) (end 30.348 30.83) (width 0.254) (layer "F.Cu") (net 13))
 (segment (start 30.348 30.83) (end 30.348 37.592) (width 0.254) (layer "F.Cu") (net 13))
 (segment (start 36.508289 36.762289) (end 31.177711 36.762289) (width 0.254) (layer "B.Cu") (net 13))
 (segment (start 37.338 37.592) (end 36.508289 36.762289) (width 0.254) (layer "B.Cu") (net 13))
 (segment (start 31.177711 36.762289) (end 30.348 37.592) (width 0.254) (layer "B.Cu") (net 13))
 (segment (start 38.074 27.432) (end 38.608 27.966) (width 0.254) (layer "F.Cu") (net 14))
 (segment (start 38.608 27.966) (end 38.608 37.592) (width 0.254) (layer "F.Cu") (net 14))
 (segment (start 34.798 25.628) (end 34.798 37.592) (width 0.254) (layer "F.Cu") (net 7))
 (segment (start 34.062 24.892) (end 34.798 25.628) (width 0.254) (layer "F.Cu") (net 7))
 (segment (start 35.464481 25.469519) (end 35.464481 36.196758) (width 0.254) (layer "F.Cu") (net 10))
 (segment (start 35.464481 36.196758) (end 36.068 36.800277) (width 0.254) (layer "F.Cu") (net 10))
 (segment (start 36.068 36.800277) (end 36.068 37.592) (width 0.254) (layer "F.Cu") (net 10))
 (segment (start 36.042 24.892) (end 35.464481 25.469519) (width 0.254) (layer "F.Cu") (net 10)))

